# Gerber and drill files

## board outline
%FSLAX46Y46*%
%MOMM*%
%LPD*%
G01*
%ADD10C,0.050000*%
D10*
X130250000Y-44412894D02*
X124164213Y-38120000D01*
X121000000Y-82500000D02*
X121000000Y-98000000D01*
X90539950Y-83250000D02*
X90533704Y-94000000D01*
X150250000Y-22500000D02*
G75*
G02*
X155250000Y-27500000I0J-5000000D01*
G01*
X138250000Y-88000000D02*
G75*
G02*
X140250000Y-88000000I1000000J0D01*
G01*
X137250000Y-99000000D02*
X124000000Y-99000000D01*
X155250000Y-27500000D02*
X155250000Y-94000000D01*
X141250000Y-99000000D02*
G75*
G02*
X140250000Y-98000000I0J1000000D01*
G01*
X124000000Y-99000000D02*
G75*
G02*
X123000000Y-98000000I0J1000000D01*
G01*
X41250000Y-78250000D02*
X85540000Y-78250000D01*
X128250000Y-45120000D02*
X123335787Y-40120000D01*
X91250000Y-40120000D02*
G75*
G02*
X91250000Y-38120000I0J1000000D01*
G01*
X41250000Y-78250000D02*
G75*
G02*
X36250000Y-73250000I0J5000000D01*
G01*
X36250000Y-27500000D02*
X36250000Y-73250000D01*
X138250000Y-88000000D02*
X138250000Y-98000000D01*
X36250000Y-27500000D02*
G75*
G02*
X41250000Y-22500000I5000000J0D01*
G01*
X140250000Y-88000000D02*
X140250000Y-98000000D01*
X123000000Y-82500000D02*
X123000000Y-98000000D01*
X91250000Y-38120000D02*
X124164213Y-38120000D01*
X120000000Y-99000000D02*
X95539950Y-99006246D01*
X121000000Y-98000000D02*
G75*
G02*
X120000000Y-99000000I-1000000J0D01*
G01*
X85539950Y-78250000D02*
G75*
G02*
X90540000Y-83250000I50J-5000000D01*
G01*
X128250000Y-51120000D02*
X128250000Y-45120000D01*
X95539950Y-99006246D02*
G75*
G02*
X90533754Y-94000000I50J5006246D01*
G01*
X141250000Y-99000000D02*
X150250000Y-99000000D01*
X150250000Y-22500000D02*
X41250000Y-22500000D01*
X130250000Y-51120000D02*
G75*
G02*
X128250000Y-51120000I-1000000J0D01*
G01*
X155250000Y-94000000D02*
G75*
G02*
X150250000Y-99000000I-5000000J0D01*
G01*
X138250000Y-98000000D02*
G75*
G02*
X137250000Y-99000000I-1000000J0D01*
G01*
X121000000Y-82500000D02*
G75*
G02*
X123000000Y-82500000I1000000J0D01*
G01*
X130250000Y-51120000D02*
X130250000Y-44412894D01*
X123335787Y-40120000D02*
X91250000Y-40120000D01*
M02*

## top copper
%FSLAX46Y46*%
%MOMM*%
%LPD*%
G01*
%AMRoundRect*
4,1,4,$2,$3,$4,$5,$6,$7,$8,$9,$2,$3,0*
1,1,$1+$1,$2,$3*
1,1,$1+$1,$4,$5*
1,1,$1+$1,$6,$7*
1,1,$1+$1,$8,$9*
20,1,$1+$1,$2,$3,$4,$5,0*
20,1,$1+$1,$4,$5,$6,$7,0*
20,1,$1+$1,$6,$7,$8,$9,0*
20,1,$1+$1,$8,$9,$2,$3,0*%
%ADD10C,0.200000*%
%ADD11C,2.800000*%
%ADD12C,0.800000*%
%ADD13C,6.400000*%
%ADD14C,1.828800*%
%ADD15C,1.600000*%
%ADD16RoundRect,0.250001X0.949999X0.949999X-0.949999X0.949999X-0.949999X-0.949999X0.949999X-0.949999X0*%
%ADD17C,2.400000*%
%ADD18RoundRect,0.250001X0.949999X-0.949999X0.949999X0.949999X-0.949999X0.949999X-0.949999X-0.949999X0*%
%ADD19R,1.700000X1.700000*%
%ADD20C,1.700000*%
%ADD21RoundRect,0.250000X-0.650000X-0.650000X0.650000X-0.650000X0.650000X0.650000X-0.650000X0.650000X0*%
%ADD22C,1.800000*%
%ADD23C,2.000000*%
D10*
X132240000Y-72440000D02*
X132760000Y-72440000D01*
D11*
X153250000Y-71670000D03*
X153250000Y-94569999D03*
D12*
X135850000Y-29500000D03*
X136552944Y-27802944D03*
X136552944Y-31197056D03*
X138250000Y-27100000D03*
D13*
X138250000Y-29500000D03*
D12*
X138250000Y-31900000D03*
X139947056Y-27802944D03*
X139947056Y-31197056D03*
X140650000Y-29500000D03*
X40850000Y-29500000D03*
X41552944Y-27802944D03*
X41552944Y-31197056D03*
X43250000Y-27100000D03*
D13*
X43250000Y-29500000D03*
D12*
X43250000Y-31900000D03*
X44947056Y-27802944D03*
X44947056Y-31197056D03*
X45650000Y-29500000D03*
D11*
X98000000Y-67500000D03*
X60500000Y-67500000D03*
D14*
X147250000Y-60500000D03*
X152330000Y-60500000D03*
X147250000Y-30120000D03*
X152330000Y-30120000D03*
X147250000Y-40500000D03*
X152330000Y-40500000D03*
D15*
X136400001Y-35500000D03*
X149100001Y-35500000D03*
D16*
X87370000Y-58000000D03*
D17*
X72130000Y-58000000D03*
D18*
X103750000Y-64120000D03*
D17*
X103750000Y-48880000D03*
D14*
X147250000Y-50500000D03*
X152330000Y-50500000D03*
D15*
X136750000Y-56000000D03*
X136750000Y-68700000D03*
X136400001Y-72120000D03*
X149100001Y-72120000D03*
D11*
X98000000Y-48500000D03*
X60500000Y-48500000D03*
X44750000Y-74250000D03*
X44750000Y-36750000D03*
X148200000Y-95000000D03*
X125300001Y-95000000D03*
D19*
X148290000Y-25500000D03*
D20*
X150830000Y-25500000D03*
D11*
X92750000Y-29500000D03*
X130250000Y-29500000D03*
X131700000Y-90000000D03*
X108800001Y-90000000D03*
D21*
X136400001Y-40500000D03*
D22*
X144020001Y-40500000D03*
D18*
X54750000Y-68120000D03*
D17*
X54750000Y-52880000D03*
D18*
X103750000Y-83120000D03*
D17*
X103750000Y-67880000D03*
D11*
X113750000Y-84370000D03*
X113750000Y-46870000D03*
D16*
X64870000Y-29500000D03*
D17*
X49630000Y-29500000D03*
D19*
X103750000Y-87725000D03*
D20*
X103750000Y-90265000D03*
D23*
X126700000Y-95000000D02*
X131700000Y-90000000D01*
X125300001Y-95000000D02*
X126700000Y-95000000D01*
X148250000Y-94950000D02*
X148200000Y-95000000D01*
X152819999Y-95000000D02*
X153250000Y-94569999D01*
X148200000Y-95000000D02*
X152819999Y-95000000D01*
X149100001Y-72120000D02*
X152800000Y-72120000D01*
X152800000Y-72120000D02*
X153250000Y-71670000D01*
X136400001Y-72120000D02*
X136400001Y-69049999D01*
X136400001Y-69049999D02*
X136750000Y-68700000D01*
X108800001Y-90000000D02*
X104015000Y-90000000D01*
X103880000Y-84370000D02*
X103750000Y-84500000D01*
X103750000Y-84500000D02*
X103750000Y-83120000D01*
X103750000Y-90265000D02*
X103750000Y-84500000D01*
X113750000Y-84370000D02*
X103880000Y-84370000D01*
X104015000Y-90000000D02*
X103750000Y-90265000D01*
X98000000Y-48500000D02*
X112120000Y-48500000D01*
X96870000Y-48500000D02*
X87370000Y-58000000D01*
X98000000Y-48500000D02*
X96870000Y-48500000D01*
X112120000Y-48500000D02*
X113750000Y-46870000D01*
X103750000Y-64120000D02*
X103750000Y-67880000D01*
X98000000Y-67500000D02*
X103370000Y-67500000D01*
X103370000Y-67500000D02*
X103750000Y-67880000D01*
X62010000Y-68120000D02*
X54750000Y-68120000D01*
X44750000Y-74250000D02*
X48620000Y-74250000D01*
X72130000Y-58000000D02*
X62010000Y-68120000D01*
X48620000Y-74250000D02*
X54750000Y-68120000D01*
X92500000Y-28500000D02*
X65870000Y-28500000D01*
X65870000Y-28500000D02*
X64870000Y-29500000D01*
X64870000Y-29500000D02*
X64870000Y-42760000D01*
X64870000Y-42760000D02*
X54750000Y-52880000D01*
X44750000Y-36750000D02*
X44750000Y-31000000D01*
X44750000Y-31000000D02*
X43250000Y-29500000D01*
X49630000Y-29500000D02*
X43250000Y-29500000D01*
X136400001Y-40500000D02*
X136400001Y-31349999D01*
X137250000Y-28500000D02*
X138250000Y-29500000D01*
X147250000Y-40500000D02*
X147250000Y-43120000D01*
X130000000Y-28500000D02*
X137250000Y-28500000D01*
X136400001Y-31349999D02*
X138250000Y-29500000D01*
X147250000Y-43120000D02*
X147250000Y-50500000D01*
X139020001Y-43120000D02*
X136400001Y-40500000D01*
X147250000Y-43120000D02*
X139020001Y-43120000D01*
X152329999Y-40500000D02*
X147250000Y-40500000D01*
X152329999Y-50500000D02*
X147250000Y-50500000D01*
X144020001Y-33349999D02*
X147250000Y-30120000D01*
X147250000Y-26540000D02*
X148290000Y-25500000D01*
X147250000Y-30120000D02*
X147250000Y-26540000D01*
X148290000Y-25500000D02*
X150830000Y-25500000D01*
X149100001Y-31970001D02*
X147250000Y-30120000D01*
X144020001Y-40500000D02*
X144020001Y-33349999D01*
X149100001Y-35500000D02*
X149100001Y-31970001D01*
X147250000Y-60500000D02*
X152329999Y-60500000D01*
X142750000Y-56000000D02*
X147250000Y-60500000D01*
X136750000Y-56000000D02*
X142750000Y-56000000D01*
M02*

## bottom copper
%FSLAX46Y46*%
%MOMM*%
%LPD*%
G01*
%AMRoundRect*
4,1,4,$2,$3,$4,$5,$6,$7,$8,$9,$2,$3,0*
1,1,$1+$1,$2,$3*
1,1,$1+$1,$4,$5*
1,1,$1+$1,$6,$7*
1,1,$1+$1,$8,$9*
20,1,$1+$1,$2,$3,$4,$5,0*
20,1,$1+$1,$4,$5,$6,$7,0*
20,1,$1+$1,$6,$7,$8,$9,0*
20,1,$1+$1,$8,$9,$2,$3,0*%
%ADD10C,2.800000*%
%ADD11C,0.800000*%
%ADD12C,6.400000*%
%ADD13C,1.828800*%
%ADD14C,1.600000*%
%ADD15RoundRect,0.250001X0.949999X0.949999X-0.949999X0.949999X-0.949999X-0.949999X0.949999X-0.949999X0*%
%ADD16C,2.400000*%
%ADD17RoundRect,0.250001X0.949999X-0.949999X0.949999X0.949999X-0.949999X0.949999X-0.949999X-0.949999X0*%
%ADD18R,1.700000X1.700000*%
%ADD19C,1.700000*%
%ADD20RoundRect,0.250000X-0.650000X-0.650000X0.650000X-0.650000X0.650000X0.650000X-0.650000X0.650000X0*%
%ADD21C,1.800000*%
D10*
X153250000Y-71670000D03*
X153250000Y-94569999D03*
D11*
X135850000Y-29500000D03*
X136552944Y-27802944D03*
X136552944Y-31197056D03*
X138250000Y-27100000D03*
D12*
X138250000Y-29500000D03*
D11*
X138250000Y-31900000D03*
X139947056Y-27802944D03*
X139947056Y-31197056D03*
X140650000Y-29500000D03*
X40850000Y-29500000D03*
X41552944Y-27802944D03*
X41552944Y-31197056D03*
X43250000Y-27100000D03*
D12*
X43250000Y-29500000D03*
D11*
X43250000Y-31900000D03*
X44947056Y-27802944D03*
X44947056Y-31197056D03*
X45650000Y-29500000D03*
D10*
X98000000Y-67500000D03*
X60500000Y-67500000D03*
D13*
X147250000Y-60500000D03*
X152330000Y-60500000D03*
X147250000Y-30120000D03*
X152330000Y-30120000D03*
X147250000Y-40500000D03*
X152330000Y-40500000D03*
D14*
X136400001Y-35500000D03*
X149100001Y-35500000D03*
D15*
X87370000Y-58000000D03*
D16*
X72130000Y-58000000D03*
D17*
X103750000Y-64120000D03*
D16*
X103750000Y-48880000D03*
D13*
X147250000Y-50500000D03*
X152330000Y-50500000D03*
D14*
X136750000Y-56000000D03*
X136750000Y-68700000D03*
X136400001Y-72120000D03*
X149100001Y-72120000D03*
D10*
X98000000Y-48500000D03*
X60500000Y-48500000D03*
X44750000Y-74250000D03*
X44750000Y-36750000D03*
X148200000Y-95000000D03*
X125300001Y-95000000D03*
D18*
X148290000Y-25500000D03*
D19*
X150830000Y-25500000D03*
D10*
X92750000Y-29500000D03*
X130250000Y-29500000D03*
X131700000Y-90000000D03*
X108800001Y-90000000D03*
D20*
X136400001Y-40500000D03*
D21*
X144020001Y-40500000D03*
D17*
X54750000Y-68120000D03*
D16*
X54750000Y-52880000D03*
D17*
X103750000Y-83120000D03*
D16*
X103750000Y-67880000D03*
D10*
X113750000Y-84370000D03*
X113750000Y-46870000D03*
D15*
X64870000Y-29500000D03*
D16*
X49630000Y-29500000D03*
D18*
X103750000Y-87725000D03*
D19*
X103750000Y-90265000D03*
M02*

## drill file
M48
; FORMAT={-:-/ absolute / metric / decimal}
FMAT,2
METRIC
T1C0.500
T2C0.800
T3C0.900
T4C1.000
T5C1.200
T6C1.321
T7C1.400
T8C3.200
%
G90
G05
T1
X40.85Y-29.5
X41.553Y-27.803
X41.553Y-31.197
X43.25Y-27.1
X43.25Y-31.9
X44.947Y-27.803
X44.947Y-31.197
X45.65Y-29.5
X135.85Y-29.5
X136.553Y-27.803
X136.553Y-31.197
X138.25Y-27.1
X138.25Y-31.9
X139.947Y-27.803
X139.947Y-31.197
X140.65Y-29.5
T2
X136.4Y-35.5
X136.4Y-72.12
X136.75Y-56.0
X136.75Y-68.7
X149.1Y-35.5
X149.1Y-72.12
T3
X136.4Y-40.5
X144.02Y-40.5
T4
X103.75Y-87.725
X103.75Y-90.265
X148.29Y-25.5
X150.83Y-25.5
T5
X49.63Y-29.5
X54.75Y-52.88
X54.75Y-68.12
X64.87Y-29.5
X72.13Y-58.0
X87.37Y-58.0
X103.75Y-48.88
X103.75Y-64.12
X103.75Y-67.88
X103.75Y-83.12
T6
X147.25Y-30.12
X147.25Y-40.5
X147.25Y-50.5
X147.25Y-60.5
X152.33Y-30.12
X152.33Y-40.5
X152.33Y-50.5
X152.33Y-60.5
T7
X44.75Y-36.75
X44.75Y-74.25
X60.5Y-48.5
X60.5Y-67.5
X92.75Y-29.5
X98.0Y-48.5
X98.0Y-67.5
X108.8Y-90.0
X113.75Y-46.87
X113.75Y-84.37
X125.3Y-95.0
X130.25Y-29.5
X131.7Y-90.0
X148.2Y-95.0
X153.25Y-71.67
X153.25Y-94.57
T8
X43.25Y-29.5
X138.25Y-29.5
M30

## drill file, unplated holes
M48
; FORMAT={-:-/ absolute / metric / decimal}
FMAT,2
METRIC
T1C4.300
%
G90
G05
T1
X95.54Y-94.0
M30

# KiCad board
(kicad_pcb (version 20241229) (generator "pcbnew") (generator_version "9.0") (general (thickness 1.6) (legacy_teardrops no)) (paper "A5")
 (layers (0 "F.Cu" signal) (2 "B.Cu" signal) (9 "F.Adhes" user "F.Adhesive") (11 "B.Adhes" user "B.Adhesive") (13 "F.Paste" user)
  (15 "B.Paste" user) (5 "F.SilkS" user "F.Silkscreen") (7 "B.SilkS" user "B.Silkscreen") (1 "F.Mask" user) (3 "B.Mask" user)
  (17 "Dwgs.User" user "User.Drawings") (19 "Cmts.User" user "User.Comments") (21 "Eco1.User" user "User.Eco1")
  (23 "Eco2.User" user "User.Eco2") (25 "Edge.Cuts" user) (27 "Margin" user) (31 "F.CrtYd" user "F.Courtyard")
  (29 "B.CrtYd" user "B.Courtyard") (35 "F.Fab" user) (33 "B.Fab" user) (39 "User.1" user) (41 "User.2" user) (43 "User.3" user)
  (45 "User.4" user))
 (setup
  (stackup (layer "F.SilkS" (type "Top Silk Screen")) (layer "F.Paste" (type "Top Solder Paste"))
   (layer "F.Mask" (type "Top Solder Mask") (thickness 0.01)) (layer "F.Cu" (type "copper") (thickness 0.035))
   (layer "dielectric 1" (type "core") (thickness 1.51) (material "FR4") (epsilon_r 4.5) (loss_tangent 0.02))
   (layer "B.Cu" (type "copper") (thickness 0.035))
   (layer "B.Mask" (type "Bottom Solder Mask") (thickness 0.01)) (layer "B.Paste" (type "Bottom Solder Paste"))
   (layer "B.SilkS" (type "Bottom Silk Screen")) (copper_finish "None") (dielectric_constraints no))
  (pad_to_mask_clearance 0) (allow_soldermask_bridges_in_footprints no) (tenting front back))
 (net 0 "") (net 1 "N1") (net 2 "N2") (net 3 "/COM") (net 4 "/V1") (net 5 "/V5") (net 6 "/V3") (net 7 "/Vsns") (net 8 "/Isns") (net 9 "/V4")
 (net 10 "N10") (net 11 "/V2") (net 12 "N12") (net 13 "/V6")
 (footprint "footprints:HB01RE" (layer "F.Cu") (at 153.25 73.12 -90)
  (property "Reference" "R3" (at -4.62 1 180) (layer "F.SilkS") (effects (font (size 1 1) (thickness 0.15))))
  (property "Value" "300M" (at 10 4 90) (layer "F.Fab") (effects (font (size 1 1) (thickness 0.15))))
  (pad "1" thru_hole circle (at -1.45 0 270) (size 2.8 2.8) (drill 1.4) (layers "*.Cu" "*.Mask") (remove_unused_layers no) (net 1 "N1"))
  (pad "2" thru_hole circle (at 21.449999 0 270) (size 2.8 2.8) (drill 1.4) (layers "*.Cu" "*.Mask") (remove_unused_layers no) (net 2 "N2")))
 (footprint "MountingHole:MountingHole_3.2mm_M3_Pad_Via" (layer "F.Cu") (at 138.25 29.5)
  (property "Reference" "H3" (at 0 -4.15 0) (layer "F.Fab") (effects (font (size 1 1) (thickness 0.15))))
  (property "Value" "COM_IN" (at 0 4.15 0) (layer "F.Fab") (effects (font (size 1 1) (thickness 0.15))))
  (pad "1" thru_hole circle (at -2.4 0) (size 0.8 0.8) (drill 0.5) (layers "*.Cu" "*.Mask") (remove_unused_layers no) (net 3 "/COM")
   (zone_connect 2))
  (pad "1" thru_hole circle (at -1.697056 -1.697056) (size 0.8 0.8) (drill 0.5) (layers "*.Cu" "*.Mask") (remove_unused_layers no)
   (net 3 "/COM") (zone_connect 2))
  (pad "1" thru_hole circle (at -1.697056 1.697056) (size 0.8 0.8) (drill 0.5) (layers "*.Cu" "*.Mask") (remove_unused_layers no)
   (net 3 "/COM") (zone_connect 2))
  (pad "1" thru_hole circle (at 0 -2.4) (size 0.8 0.8) (drill 0.5) (layers "*.Cu" "*.Mask") (remove_unused_layers no) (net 3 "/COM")
   (zone_connect 2))
  (pad "1" thru_hole circle (at 0 0) (size 6.4 6.4) (drill 3.2) (layers "*.Cu" "*.Mask") (remove_unused_layers no) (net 3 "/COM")
   (zone_connect 2))
  (pad "1" thru_hole circle (at 0 2.4) (size 0.8 0.8) (drill 0.5) (layers "*.Cu" "*.Mask") (remove_unused_layers no) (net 3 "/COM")
   (zone_connect 2))
  (pad "1" thru_hole circle (at 1.697056 -1.697056) (size 0.8 0.8) (drill 0.5) (layers "*.Cu" "*.Mask") (remove_unused_layers no)
   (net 3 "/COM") (zone_connect 2))
  (pad "1" thru_hole circle (at 1.697056 1.697056) (size 0.8 0.8) (drill 0.5) (layers "*.Cu" "*.Mask") (remove_unused_layers no)
   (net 3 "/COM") (zone_connect 2))
  (pad "1" thru_hole circle (at 2.4 0) (size 0.8 0.8) (drill 0.5) (layers "*.Cu" "*.Mask") (remove_unused_layers no) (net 3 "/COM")
   (zone_connect 2)))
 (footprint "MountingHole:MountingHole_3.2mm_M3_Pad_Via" (layer "F.Cu") (at 43.25 29.5)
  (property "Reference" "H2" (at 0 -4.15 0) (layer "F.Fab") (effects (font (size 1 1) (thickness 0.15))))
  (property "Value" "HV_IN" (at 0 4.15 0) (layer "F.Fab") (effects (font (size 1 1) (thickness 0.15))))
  (pad "1" thru_hole circle (at -2.4 0) (size 0.8 0.8) (drill 0.5) (layers "*.Cu" "*.Mask") (remove_unused_layers no) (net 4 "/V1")
   (zone_connect 2))
  (pad "1" thru_hole circle (at -1.697056 -1.697056) (size 0.8 0.8) (drill 0.5) (layers "*.Cu" "*.Mask") (remove_unused_layers no)
   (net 4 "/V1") (zone_connect 2))
  (pad "1" thru_hole circle (at -1.697056 1.697056) (size 0.8 0.8) (drill 0.5) (layers "*.Cu" "*.Mask") (remove_unused_layers no)
   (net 4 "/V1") (zone_connect 2))
  (pad "1" thru_hole circle (at 0 -2.4) (size 0.8 0.8) (drill 0.5) (layers "*.Cu" "*.Mask") (remove_unused_layers no) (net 4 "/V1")
   (zone_connect 2))
  (pad "1" thru_hole circle (at 0 0) (size 6.4 6.4) (drill 3.2) (layers "*.Cu" "*.Mask") (remove_unused_layers no) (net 4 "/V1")
   (zone_connect 2))
  (pad "1" thru_hole circle (at 0 2.4) (size 0.8 0.8) (drill 0.5) (layers "*.Cu" "*.Mask") (remove_unused_layers no) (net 4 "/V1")
   (zone_connect 2))
  (pad "1" thru_hole circle (at 1.697056 -1.697056) (size 0.8 0.8) (drill 0.5) (layers "*.Cu" "*.Mask") (remove_unused_layers no)
   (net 4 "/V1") (zone_connect 2))
  (pad "1" thru_hole circle (at 1.697056 1.697056) (size 0.8 0.8) (drill 0.5) (layers "*.Cu" "*.Mask") (remove_unused_layers no)
   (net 4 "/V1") (zone_connect 2))
  (pad "1" thru_hole circle (at 2.4 0) (size 0.8 0.8) (drill 0.5) (layers "*.Cu" "*.Mask") (remove_unused_layers no) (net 4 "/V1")
   (zone_connect 2)))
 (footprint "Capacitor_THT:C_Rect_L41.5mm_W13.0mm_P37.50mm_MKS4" (layer "F.Cu") (at 98 67.5 180)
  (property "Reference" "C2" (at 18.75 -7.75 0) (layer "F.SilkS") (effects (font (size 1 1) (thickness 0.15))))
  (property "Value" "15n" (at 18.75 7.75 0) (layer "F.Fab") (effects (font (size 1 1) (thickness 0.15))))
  (pad "1" thru_hole circle (at 0 0 180) (size 2.8 2.8) (drill 1.4) (layers "*.Cu" "*.Mask") (remove_unused_layers no) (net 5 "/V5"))
  (pad "2" thru_hole circle (at 37.5 0 180) (size 2.8 2.8) (drill 1.4) (layers "*.Cu" "*.Mask") (remove_unused_layers no) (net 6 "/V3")))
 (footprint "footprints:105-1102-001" (layer "F.Cu") (at 147.25 60.5)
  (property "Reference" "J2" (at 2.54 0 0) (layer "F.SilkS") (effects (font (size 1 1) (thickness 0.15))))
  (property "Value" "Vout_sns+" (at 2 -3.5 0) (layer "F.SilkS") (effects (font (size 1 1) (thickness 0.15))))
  (pad "1" thru_hole circle (at 0 0) (size 1.8288 1.8288) (drill 1.3208) (layers "*.Cu" "*.Mask") (remove_unused_layers no) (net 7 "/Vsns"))
  (pad "2" thru_hole circle (at 5.08 0) (size 1.8288 1.8288) (drill 1.3208) (layers "*.Cu" "*.Mask") (remove_unused_layers no)
   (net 7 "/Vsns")))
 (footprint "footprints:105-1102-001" (layer "F.Cu") (at 147.25 30.12)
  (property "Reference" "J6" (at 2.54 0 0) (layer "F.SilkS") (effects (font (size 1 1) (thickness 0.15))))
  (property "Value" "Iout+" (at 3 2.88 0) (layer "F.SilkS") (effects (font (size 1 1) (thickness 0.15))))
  (pad "1" thru_hole circle (at 0 0) (size 1.8288 1.8288) (drill 1.3208) (layers "*.Cu" "*.Mask") (remove_unused_layers no) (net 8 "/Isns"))
  (pad "2" thru_hole circle (at 5.08 0) (size 1.8288 1.8288) (drill 1.3208) (layers "*.Cu" "*.Mask") (remove_unused_layers no)
   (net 8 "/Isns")))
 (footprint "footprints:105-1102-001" (layer "F.Cu") (at 147.25 40.5)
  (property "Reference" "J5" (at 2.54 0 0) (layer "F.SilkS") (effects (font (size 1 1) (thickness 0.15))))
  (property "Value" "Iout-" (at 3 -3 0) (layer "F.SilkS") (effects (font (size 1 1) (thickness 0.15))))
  (pad "1" thru_hole circle (at 0 0) (size 1.8288 1.8288) (drill 1.3208) (layers "*.Cu" "*.Mask") (remove_unused_layers no) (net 3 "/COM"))
  (pad "2" thru_hole circle (at 5.08 0) (size 1.8288 1.8288) (drill 1.3208) (layers "*.Cu" "*.Mask") (remove_unused_layers no)
   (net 3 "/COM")))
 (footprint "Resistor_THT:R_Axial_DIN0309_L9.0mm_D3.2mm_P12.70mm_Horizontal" (layer "F.Cu") (at 136.400001 35.5)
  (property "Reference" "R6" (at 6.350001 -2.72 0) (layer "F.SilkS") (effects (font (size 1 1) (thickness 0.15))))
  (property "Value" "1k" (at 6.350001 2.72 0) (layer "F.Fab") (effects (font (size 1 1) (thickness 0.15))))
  (pad "1" thru_hole circle (at 0 0) (size 1.6 1.6) (drill 0.8) (layers "*.Cu" "*.Mask") (remove_unused_layers no) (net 3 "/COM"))
  (pad "2" thru_hole circle (at 12.7 0) (size 1.6 1.6) (drill 0.8) (layers "*.Cu" "*.Mask") (remove_unused_layers no) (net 8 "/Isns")))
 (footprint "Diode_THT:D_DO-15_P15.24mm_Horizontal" (layer "F.Cu") (at 87.37 58 180)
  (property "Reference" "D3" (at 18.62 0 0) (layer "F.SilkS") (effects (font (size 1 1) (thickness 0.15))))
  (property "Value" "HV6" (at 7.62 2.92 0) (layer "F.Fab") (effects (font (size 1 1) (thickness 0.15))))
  (pad "1" thru_hole roundrect (at 0 0 180) (size 2.4 2.4) (drill 1.2) (layers "*.Cu" "*.Mask") (remove_unused_layers no)
   (roundrect_rratio 0.104167) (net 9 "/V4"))
  (pad "2" thru_hole circle (at 15.24 0 180) (size 2.4 2.4) (drill 1.2) (layers "*.Cu" "*.Mask") (remove_unused_layers no) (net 6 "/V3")))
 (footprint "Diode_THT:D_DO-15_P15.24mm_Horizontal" (layer "F.Cu") (at 103.75 64.12 90)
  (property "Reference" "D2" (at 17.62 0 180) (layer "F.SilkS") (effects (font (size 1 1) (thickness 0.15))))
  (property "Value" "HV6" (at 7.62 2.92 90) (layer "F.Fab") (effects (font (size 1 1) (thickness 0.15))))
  (pad "1" thru_hole roundrect (at 0 0 90) (size 2.4 2.4) (drill 1.2) (layers "*.Cu" "*.Mask") (remove_unused_layers no)
   (roundrect_rratio 0.104167) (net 5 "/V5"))
  (pad "2" thru_hole circle (at 15.24 0 90) (size 2.4 2.4) (drill 1.2) (layers "*.Cu" "*.Mask") (remove_unused_layers no) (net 9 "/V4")))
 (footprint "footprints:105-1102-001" (layer "F.Cu") (at 147.25 50.5)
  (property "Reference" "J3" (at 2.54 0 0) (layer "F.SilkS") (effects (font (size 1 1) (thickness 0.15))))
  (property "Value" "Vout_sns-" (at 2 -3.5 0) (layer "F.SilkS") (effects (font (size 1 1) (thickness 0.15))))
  (pad "1" thru_hole circle (at 0 0) (size 1.8288 1.8288) (drill 1.3208) (layers "*.Cu" "*.Mask") (remove_unused_layers no) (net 3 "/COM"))
  (pad "2" thru_hole circle (at 5.08 0) (size 1.8288 1.8288) (drill 1.3208) (layers "*.Cu" "*.Mask") (remove_unused_layers no)
   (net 3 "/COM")))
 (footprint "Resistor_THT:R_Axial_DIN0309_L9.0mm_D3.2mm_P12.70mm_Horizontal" (layer "F.Cu") (at 136.75 56 -90)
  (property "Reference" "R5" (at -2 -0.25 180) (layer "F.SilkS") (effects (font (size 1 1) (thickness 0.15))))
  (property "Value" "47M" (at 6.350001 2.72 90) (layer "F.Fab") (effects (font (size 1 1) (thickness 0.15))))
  (pad "1" thru_hole circle (at 0 0 270) (size 1.6 1.6) (drill 0.8) (layers "*.Cu" "*.Mask") (remove_unused_layers no) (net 7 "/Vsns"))
  (pad "2" thru_hole circle (at 12.7 0 270) (size 1.6 1.6) (drill 0.8) (layers "*.Cu" "*.Mask") (remove_unused_layers no) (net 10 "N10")))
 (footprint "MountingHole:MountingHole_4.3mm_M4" (layer "F.Cu") (at 95.53995 94)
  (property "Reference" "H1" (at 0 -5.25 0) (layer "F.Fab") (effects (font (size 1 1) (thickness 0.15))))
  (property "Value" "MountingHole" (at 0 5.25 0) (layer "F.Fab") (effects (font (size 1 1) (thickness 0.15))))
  (pad "" np_thru_hole circle (at 0 0) (size 4.3 4.3) (drill 4.3) (layers "*.Cu" "*.Mask")))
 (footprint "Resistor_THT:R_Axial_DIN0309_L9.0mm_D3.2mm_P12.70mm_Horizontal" (layer "F.Cu") (at 136.400001 72.12)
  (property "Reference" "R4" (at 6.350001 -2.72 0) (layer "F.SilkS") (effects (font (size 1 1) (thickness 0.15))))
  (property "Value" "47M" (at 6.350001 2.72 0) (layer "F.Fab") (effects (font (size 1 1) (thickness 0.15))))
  (pad "1" thru_hole circle (at 0 0) (size 1.6 1.6) (drill 0.8) (layers "*.Cu" "*.Mask") (remove_unused_layers no) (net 10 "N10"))
  (pad "2" thru_hole circle (at 12.7 0) (size 1.6 1.6) (drill 0.8) (layers "*.Cu" "*.Mask") (remove_unused_layers no) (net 1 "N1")))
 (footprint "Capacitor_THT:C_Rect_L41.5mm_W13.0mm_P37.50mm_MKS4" (layer "F.Cu") (at 98 48.5 180)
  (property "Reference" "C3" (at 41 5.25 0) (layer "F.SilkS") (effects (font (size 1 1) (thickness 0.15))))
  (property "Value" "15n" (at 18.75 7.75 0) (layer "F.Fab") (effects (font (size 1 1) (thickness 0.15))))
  (pad "1" thru_hole circle (at 0 0 180) (size 2.8 2.8) (drill 1.4) (layers "*.Cu" "*.Mask") (remove_unused_layers no) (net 9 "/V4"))
  (pad "2" thru_hole circle (at 37.5 0 180) (size 2.8 2.8) (drill 1.4) (layers "*.Cu" "*.Mask") (remove_unused_layers no) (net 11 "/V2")))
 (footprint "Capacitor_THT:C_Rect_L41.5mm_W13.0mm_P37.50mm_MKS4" (layer "F.Cu") (at 44.75 74.25 90)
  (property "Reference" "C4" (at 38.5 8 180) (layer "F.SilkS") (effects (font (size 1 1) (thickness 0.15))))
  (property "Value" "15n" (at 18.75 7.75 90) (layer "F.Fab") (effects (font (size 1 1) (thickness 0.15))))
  (pad "1" thru_hole circle (at 0 0 90) (size 2.8 2.8) (drill 1.4) (layers "*.Cu" "*.Mask") (remove_unused_layers no) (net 6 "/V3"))
  (pad "2" thru_hole circle (at 37.5 0 90) (size 2.8 2.8) (drill 1.4) (layers "*.Cu" "*.Mask") (remove_unused_layers no) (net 4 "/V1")))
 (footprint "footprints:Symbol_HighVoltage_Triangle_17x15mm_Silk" (layer "F.Cu") (at 132.5 78.5)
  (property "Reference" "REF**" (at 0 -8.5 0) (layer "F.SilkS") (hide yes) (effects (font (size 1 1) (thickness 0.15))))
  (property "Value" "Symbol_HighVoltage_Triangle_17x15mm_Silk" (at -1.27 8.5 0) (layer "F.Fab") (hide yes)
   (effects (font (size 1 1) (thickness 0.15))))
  (fp_line (start -0.26 -6.06) (end 0.26 -6.06) (stroke (width 0.2) (type default)) (layer "F.Cu")))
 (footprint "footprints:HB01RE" (layer "F.Cu") (at 146.75 95 180)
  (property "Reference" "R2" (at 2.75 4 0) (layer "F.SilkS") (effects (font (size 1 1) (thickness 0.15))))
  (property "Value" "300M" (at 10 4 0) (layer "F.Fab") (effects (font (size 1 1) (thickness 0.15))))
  (pad "1" thru_hole circle (at -1.45 0 180) (size 2.8 2.8) (drill 1.4) (layers "*.Cu" "*.Mask") (remove_unused_layers no) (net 2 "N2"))
  (pad "2" thru_hole circle (at 21.449999 0 180) (size 2.8 2.8) (drill 1.4) (layers "*.Cu" "*.Mask") (remove_unused_layers no)
   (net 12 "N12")))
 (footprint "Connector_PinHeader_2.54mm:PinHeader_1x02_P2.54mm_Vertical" (layer "F.Cu") (at 148.29 25.5 90)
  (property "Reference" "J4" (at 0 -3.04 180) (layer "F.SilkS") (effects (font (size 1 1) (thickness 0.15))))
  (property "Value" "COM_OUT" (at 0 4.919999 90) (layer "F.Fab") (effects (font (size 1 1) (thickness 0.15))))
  (pad "1" thru_hole rect (at 0 0 90) (size 1.7 1.7) (drill 1) (layers "*.Cu" "*.Mask") (remove_unused_layers no) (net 8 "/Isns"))
  (pad "2" thru_hole circle (at 0 2.54 90) (size 1.7 1.7) (drill 1) (layers "*.Cu" "*.Mask") (remove_unused_layers no) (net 8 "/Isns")))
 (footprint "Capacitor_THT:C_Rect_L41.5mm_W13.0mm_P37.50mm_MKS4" (layer "F.Cu") (at 92.75 29.5)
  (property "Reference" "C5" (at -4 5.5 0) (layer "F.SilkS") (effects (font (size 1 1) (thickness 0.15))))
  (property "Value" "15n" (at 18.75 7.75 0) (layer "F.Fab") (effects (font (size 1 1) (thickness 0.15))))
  (pad "1" thru_hole circle (at 0 0) (size 2.8 2.8) (drill 1.4) (layers "*.Cu" "*.Mask") (remove_unused_layers no) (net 11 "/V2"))
  (pad "2" thru_hole circle (at 37.5 0) (size 2.8 2.8) (drill 1.4) (layers "*.Cu" "*.Mask") (remove_unused_layers no) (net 3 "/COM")))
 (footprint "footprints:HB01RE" (layer "F.Cu") (at 130.25 90 180)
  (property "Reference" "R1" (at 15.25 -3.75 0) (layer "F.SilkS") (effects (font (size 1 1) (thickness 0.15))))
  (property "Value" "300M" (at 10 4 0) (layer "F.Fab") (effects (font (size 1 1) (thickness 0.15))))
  (pad "1" thru_hole circle (at -1.45 0 180) (size 2.8 2.8) (drill 1.4) (layers "*.Cu" "*.Mask") (remove_unused_layers no) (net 12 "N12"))
  (pad "2" thru_hole circle (at 21.449999 0 180) (size 2.8 2.8) (drill 1.4) (layers "*.Cu" "*.Mask") (remove_unused_layers no)
   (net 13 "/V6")))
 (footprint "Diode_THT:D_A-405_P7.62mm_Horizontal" (layer "F.Cu") (at 136.400001 40.5)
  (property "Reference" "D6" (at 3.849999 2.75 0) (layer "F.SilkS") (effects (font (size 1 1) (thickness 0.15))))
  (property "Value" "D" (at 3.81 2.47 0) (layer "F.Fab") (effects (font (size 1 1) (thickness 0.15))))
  (pad "1" thru_hole roundrect (at 0 0) (size 1.8 1.8) (drill 0.9) (layers "*.Cu" "*.Mask") (remove_unused_layers no)
   (roundrect_rratio 0.138889) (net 3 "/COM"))
  (pad "2" thru_hole circle (at 7.62 0) (size 1.8 1.8) (drill 0.9) (layers "*.Cu" "*.Mask") (remove_unused_layers no) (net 8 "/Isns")))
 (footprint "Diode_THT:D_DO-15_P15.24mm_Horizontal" (layer "F.Cu") (at 54.75 68.12 90)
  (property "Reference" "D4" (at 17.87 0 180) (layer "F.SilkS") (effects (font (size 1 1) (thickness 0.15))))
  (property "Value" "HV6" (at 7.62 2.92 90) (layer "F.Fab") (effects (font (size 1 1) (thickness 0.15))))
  (pad "1" thru_hole roundrect (at 0 0 90) (size 2.4 2.4) (drill 1.2) (layers "*.Cu" "*.Mask") (remove_unused_layers no)
   (roundrect_rratio 0.104167) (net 6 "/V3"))
  (pad "2" thru_hole circle (at 15.24 0 90) (size 2.4 2.4) (drill 1.2) (layers "*.Cu" "*.Mask") (remove_unused_layers no) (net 11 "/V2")))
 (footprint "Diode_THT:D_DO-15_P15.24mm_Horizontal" (layer "F.Cu") (at 103.75 83.12 90)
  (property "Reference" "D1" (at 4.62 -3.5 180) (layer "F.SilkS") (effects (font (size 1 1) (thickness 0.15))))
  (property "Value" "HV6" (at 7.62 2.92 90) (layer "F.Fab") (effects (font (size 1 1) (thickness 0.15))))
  (pad "1" thru_hole roundrect (at 0 0 90) (size 2.4 2.4) (drill 1.2) (layers "*.Cu" "*.Mask") (remove_unused_layers no)
   (roundrect_rratio 0.104167) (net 13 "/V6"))
  (pad "2" thru_hole circle (at 15.24 0 90) (size 2.4 2.4) (drill 1.2) (layers "*.Cu" "*.Mask") (remove_unused_layers no) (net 5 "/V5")))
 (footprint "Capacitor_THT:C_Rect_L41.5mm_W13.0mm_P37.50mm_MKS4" (layer "F.Cu") (at 113.75 84.37 90)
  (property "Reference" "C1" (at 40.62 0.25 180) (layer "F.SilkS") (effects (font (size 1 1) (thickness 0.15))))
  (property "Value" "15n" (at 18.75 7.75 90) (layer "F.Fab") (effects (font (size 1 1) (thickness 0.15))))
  (pad "1" thru_hole circle (at 0 0 90) (size 2.8 2.8) (drill 1.4) (layers "*.Cu" "*.Mask") (remove_unused_layers no) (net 13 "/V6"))
  (pad "2" thru_hole circle (at 37.5 0 90) (size 2.8 2.8) (drill 1.4) (layers "*.Cu" "*.Mask") (remove_unused_layers no) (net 9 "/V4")))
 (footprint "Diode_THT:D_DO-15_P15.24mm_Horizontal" (layer "F.Cu") (at 64.87 29.5 180)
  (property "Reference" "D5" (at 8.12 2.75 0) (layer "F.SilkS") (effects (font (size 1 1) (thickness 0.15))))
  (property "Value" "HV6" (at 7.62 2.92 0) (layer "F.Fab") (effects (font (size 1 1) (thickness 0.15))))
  (pad "1" thru_hole roundrect (at 0 0 180) (size 2.4 2.4) (drill 1.2) (layers "*.Cu" "*.Mask") (remove_unused_layers no)
   (roundrect_rratio 0.104167) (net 11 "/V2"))
  (pad "2" thru_hole circle (at 15.24 0 180) (size 2.4 2.4) (drill 1.2) (layers "*.Cu" "*.Mask") (remove_unused_layers no) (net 4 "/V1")))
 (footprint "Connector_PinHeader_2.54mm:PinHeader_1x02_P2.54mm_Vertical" (layer "F.Cu") (at 103.75 87.725)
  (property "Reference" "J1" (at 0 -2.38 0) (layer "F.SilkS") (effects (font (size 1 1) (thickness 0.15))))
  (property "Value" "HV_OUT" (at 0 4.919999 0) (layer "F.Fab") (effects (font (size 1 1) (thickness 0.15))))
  (pad "1" thru_hole rect (at 0 0) (size 1.7 1.7) (drill 1) (layers "*.Cu" "*.Mask") (remove_unused_layers no) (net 13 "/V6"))
  (pad "2" thru_hole circle (at 0 2.54) (size 1.7 1.7) (drill 1) (layers "*.Cu" "*.Mask") (remove_unused_layers no) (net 13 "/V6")))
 (gr_line (start 130.25 44.412894) (end 124.164213 38.12) (stroke (width 0.05) (type default)) (layer "Edge.Cuts"))
 (gr_line (start 121 82.5) (end 121 98) (stroke (width 0.05) (type default)) (layer "Edge.Cuts"))
 (gr_line (start 90.53995 83.25) (end 90.533704 94) (stroke (width 0.05) (type default)) (layer "Edge.Cuts"))
 (gr_arc (start 150.25 22.5) (mid 153.785534 23.964466) (end 155.25 27.5) (stroke (width 0.05) (type default)) (layer "Edge.Cuts"))
 (gr_arc (start 138.25 88) (mid 139.25 87) (end 140.25 88) (stroke (width 0.05) (type default)) (layer "Edge.Cuts"))
 (gr_line (start 137.25 99) (end 124 99) (stroke (width 0.05) (type default)) (layer "Edge.Cuts"))
 (gr_line (start 155.25 27.5) (end 155.25 94) (stroke (width 0.05) (type default)) (layer "Edge.Cuts"))
 (gr_arc (start 141.25 99) (mid 140.542893 98.707107) (end 140.25 98) (stroke (width 0.05) (type default)) (layer "Edge.Cuts"))
 (gr_arc (start 124 99) (mid 123.292893 98.707107) (end 123 98) (stroke (width 0.05) (type default)) (layer "Edge.Cuts"))
 (gr_line (start 41.25 78.25) (end 85.54 78.25) (stroke (width 0.05) (type default)) (layer "Edge.Cuts"))
 (gr_line (start 128.25 45.12) (end 123.335787 40.12) (stroke (width 0.05) (type default)) (layer "Edge.Cuts"))
 (gr_arc (start 91.25 40.12) (mid 90.25 39.12) (end 91.25 38.12) (stroke (width 0.05) (type default)) (layer "Edge.Cuts"))
 (gr_arc (start 41.25 78.25) (mid 37.714466 76.785534) (end 36.25 73.25) (stroke (width 0.05) (type default)) (layer "Edge.Cuts"))
 (gr_line (start 36.25 27.5) (end 36.25 73.25) (stroke (width 0.05) (type default)) (layer "Edge.Cuts"))
 (gr_line (start 138.25 88) (end 138.25 98) (stroke (width 0.05) (type default)) (layer "Edge.Cuts"))
 (gr_arc (start 36.25 27.5) (mid 37.714466 23.964466) (end 41.25 22.5) (stroke (width 0.05) (type default)) (layer "Edge.Cuts"))
 (gr_line (start 140.25 88) (end 140.25 98) (stroke (width 0.05) (type default)) (layer "Edge.Cuts"))
 (gr_line (start 123 82.5) (end 123 98) (stroke (width 0.05) (type default)) (layer "Edge.Cuts"))
 (gr_line (start 91.25 38.12) (end 124.164213 38.12) (stroke (width 0.05) (type default)) (layer "Edge.Cuts"))
 (gr_line (start 120 99) (end 95.53995 99.006246) (stroke (width 0.05) (type default)) (layer "Edge.Cuts"))
 (gr_arc (start 121 98) (mid 120.707107 98.707107) (end 120 99) (stroke (width 0.05) (type default)) (layer "Edge.Cuts"))
 (gr_arc (start 85.53995 78.25) (mid 89.075484 79.714466) (end 90.53995 83.25) (stroke (width 0.05) (type default)) (layer "Edge.Cuts"))
 (gr_line (start 128.25 51.12) (end 128.25 45.12) (stroke (width 0.05) (type default)) (layer "Edge.Cuts"))
 (gr_arc (start 95.53995 99.006246) (mid 92 97.53995) (end 90.533704 94) (stroke (width 0.05) (type default)) (layer "Edge.Cuts"))
 (gr_line (start 141.25 99) (end 150.25 99) (stroke (width 0.05) (type default)) (layer "Edge.Cuts"))
 (gr_line (start 150.25 22.5) (end 41.25 22.5) (stroke (width 0.05) (type default)) (layer "Edge.Cuts"))
 (gr_arc (start 130.25 51.12) (mid 129.25 52.12) (end 128.25 51.12) (stroke (width 0.05) (type default)) (layer "Edge.Cuts"))
 (gr_arc (start 155.25 94) (mid 153.785534 97.535534) (end 150.25 99) (stroke (width 0.05) (type default)) (layer "Edge.Cuts"))
 (gr_arc (start 138.25 98) (mid 137.957107 98.707107) (end 137.25 99) (stroke (width 0.05) (type default)) (layer "Edge.Cuts"))
 (gr_arc (start 121 82.5) (mid 122 81.5) (end 123 82.5) (stroke (width 0.05) (type default)) (layer "Edge.Cuts"))
 (gr_line (start 130.25 51.12) (end 130.25 44.412894) (stroke (width 0.05) (type default)) (layer "Edge.Cuts"))
 (gr_line (start 123.335787 40.12) (end 91.25 40.12) (stroke (width 0.05) (type default)) (layer "Edge.Cuts"))
 (segment (start 126.7 95) (end 131.7 90) (width 2) (layer "F.Cu") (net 12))
 (segment (start 125.300001 95) (end 126.7 95) (width 2) (layer "F.Cu") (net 12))
 (segment (start 148.25 94.95) (end 148.2 95) (width 2) (layer "F.Cu") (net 2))
 (segment (start 152.819999 95) (end 153.25 94.569999) (width 2) (layer "F.Cu") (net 2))
 (segment (start 148.2 95) (end 152.819999 95) (width 2) (layer "F.Cu") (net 2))
 (segment (start 149.100001 72.12) (end 152.8 72.12) (width 2) (layer "F.Cu") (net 1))
 (segment (start 152.8 72.12) (end 153.25 71.67) (width 2) (layer "F.Cu") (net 1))
 (segment (start 136.400001 72.12) (end 136.400001 69.049999) (width 2) (layer "F.Cu") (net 10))
 (segment (start 136.400001 69.049999) (end 136.75 68.7) (width 2) (layer "F.Cu") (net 10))
 (segment (start 108.800001 90) (end 104.015 90) (width 2) (layer "F.Cu") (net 13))
 (segment (start 103.88 84.37) (end 103.75 84.5) (width 2) (layer "F.Cu") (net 13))
 (segment (start 103.75 84.5) (end 103.75 83.12) (width 2) (layer "F.Cu") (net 13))
 (segment (start 103.75 90.265) (end 103.75 84.5) (width 2) (layer "F.Cu") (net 13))
 (segment (start 113.75 84.37) (end 103.88 84.37) (width 2) (layer "F.Cu") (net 13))
 (segment (start 104.015 90) (end 103.75 90.265) (width 2) (layer "F.Cu") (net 13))
 (segment (start 98 48.5) (end 112.12 48.5) (width 2) (layer "F.Cu") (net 9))
 (segment (start 96.87 48.5) (end 87.37 58) (width 2) (layer "F.Cu") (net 9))
 (segment (start 98 48.5) (end 96.87 48.5) (width 2) (layer "F.Cu") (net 9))
 (segment (start 112.12 48.5) (end 113.75 46.87) (width 2) (layer "F.Cu") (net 9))
 (segment (start 103.75 64.12) (end 103.75 67.88) (width 2) (layer "F.Cu") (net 5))
 (segment (start 98 67.5) (end 103.37 67.5) (width 2) (layer "F.Cu") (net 5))
 (segment (start 103.37 67.5) (end 103.75 67.88) (width 2) (layer "F.Cu") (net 5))
 (segment (start 62.01 68.12) (end 54.75 68.12) (width 2) (layer "F.Cu") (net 6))
 (segment (start 44.75 74.25) (end 48.62 74.25) (width 2) (layer "F.Cu") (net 6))
 (segment (start 72.13 58) (end 62.01 68.12) (width 2) (layer "F.Cu") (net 6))
 (segment (start 48.62 74.25) (end 54.75 68.12) (width 2) (layer "F.Cu") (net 6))
 (segment (start 92.5 28.5) (end 65.87 28.5) (width 2) (layer "F.Cu") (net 11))
 (segment (start 65.87 28.5) (end 64.87 29.5) (width 2) (layer "F.Cu") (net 11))
 (segment (start 64.87 29.5) (end 64.87 42.76) (width 2) (layer "F.Cu") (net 11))
 (segment (start 64.87 42.76) (end 54.75 52.88) (width 2) (layer "F.Cu") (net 11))
 (segment (start 44.75 36.75) (end 44.75 31) (width 2) (layer "F.Cu") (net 4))
 (segment (start 44.75 31) (end 43.25 29.5) (width 2) (layer "F.Cu") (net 4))
 (segment (start 49.63 29.5) (end 43.25 29.5) (width 2) (layer "F.Cu") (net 4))
 (segment (start 136.400001 40.5) (end 136.400001 31.349999) (width 2) (layer "F.Cu") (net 3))
 (segment (start 137.25 28.5) (end 138.25 29.5) (width 2) (layer "F.Cu") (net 3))
 (segment (start 147.25 40.5) (end 147.25 43.12) (width 2) (layer "F.Cu") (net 3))
 (segment (start 130 28.5) (end 137.25 28.5) (width 2) (layer "F.Cu") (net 3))
 (segment (start 136.400001 31.349999) (end 138.25 29.5) (width 2) (layer "F.Cu") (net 3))
 (segment (start 147.25 43.12) (end 147.25 50.5) (width 2) (layer "F.Cu") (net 3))
 (segment (start 139.020001 43.12) (end 136.400001 40.5) (width 2) (layer "F.Cu") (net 3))
 (segment (start 147.25 43.12) (end 139.020001 43.12) (width 2) (layer "F.Cu") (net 3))
 (segment (start 152.329999 40.5) (end 147.25 40.5) (width 2) (layer "F.Cu") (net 3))
 (segment (start 152.329999 50.5) (end 147.25 50.5) (width 2) (layer "F.Cu") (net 3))
 (segment (start 144.020001 33.349999) (end 147.25 30.12) (width 2) (layer "F.Cu") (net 8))
 (segment (start 147.25 26.54) (end 148.29 25.5) (width 2) (layer "F.Cu") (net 8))
 (segment (start 147.25 30.12) (end 147.25 26.54) (width 2) (layer "F.Cu") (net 8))
 (segment (start 148.29 25.5) (end 150.83 25.5) (width 2) (layer "F.Cu") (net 8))
 (segment (start 149.100001 31.970001) (end 147.25 30.12) (width 2) (layer "F.Cu") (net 8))
 (segment (start 144.020001 40.5) (end 144.020001 33.349999) (width 2) (layer "F.Cu") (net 8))
 (segment (start 149.100001 35.5) (end 149.100001 31.970001) (width 2) (layer "F.Cu") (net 8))
 (segment (start 147.25 60.5) (end 152.329999 60.5) (width 2) (layer "F.Cu") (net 7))
 (segment (start 142.75 56) (end 147.25 60.5) (width 2) (layer "F.Cu") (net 7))
 (segment (start 136.75 56) (end 142.75 56) (width 2) (layer "F.Cu") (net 7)))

